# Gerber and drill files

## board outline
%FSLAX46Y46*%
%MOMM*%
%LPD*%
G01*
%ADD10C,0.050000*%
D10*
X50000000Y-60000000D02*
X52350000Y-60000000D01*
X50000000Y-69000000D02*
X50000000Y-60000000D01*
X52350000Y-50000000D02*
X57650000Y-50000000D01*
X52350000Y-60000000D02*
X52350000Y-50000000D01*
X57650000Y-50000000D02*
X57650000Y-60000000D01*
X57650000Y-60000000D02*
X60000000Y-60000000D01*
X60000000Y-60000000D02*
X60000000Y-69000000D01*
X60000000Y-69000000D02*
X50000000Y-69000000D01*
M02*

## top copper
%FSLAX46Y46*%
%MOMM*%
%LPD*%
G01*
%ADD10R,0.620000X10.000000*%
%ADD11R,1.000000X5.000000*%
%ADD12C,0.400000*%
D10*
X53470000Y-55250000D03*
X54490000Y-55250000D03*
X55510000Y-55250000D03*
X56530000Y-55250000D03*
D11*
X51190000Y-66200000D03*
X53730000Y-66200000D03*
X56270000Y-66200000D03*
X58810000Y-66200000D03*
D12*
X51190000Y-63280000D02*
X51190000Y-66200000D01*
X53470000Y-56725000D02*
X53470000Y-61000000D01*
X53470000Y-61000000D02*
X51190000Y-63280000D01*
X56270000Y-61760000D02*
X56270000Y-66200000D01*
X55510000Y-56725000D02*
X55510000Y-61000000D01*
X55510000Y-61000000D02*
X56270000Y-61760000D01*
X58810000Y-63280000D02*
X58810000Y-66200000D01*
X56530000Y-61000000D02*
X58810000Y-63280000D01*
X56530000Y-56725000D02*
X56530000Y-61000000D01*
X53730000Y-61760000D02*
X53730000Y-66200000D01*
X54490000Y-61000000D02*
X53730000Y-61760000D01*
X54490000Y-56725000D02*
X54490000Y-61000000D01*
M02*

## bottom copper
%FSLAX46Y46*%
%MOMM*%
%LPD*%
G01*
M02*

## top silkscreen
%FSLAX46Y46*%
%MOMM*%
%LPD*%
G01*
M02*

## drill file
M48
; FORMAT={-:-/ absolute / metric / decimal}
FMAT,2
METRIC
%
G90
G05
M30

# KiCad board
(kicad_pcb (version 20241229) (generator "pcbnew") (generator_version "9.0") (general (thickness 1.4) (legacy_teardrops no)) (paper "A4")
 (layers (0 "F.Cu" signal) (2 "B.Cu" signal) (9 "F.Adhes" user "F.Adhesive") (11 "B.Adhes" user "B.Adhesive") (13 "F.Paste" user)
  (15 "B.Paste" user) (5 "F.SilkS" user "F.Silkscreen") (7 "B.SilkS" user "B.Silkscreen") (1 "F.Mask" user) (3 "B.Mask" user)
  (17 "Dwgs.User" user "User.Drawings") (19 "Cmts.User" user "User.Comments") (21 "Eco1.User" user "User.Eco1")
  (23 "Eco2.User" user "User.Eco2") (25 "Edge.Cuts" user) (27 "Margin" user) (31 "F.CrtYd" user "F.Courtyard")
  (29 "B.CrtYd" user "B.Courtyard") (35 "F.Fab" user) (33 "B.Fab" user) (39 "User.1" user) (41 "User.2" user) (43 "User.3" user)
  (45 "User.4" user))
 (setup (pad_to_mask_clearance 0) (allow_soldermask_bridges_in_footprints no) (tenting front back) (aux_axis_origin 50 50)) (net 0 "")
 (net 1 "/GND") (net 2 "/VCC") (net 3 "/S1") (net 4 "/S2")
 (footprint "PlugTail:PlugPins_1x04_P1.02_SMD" (layer "F.Cu") (at 55 50)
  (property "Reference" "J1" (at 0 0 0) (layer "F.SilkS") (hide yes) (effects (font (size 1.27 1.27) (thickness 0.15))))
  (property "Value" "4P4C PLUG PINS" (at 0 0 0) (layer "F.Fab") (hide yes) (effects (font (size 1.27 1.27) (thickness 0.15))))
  (pad "1" smd rect (at -1.53 5.25) (size 0.62 10) (layers "F.Cu" "F.Mask") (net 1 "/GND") (thermal_bridge_angle 45))
  (pad "2" smd rect (at -0.51 5.25) (size 0.62 10) (layers "F.Cu" "F.Mask") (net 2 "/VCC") (thermal_bridge_angle 45))
  (pad "3" smd rect (at 0.51 5.25) (size 0.62 10) (layers "F.Cu" "F.Mask") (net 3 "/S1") (thermal_bridge_angle 45))
  (pad "4" smd rect (at 1.53 5.25) (size 0.62 10) (layers "F.Cu" "F.Mask") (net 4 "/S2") (thermal_bridge_angle 45)))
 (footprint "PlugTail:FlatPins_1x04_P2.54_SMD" (layer "F.Cu") (at 55 66.2)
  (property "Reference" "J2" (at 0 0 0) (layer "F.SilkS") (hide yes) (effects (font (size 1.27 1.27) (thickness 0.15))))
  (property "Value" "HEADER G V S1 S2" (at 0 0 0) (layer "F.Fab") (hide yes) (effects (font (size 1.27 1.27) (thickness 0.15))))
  (pad "1" smd rect (at -3.81 0) (size 1 5) (layers "F.Cu" "F.Mask") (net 1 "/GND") (thermal_bridge_angle 45))
  (pad "2" smd rect (at -1.27 0) (size 1 5) (layers "F.Cu" "F.Mask") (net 2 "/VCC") (thermal_bridge_angle 45))
  (pad "3" smd rect (at 1.27 0) (size 1 5) (layers "F.Cu" "F.Mask") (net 3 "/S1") (thermal_bridge_angle 45))
  (pad "4" smd rect (at 3.81 0) (size 1 5) (layers "F.Cu" "F.Mask") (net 4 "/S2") (thermal_bridge_angle 45)))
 (gr_line (start 50 60) (end 52.35 60) (stroke (width 0.05) (type default)) (layer "Edge.Cuts"))
 (gr_line (start 50 69) (end 50 60) (stroke (width 0.05) (type default)) (layer "Edge.Cuts"))
 (gr_line (start 52.35 50) (end 57.65 50) (stroke (width 0.05) (type default)) (layer "Edge.Cuts"))
 (gr_line (start 52.35 60) (end 52.35 50) (stroke (width 0.05) (type default)) (layer "Edge.Cuts"))
 (gr_line (start 57.65 50) (end 57.65 60) (stroke (width 0.05) (type default)) (layer "Edge.Cuts"))
 (gr_line (start 57.65 60) (end 60 60) (stroke (width 0.05) (type default)) (layer "Edge.Cuts"))
 (gr_line (start 60 60) (end 60 69) (stroke (width 0.05) (type default)) (layer "Edge.Cuts"))
 (gr_line (start 60 69) (end 50 69) (stroke (width 0.05) (type default)) (layer "Edge.Cuts"))
 (segment (start 51.19 63.28) (end 51.19 66.2) (width 0.4) (layer "F.Cu") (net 1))
 (segment (start 53.47 56.725) (end 53.47 61) (width 0.4) (layer "F.Cu") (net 1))
 (segment (start 53.47 61) (end 51.19 63.28) (width 0.4) (layer "F.Cu") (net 1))
 (segment (start 56.27 61.76) (end 56.27 66.2) (width 0.4) (layer "F.Cu") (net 3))
 (segment (start 55.51 56.725) (end 55.51 61) (width 0.4) (layer "F.Cu") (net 3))
 (segment (start 55.51 61) (end 56.27 61.76) (width 0.4) (layer "F.Cu") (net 3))
 (segment (start 58.81 63.28) (end 58.81 66.2) (width 0.4) (layer "F.Cu") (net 4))
 (segment (start 56.53 61) (end 58.81 63.28) (width 0.4) (layer "F.Cu") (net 4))
 (segment (start 56.53 56.725) (end 56.53 61) (width 0.4) (layer "F.Cu") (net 4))
 (segment (start 53.73 61.76) (end 53.73 66.2) (width 0.4) (layer "F.Cu") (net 2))
 (segment (start 54.49 61) (end 53.73 61.76) (width 0.4) (layer "F.Cu") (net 2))
 (segment (start 54.49 56.725) (end 54.49 61) (width 0.4) (layer "F.Cu") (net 2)))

